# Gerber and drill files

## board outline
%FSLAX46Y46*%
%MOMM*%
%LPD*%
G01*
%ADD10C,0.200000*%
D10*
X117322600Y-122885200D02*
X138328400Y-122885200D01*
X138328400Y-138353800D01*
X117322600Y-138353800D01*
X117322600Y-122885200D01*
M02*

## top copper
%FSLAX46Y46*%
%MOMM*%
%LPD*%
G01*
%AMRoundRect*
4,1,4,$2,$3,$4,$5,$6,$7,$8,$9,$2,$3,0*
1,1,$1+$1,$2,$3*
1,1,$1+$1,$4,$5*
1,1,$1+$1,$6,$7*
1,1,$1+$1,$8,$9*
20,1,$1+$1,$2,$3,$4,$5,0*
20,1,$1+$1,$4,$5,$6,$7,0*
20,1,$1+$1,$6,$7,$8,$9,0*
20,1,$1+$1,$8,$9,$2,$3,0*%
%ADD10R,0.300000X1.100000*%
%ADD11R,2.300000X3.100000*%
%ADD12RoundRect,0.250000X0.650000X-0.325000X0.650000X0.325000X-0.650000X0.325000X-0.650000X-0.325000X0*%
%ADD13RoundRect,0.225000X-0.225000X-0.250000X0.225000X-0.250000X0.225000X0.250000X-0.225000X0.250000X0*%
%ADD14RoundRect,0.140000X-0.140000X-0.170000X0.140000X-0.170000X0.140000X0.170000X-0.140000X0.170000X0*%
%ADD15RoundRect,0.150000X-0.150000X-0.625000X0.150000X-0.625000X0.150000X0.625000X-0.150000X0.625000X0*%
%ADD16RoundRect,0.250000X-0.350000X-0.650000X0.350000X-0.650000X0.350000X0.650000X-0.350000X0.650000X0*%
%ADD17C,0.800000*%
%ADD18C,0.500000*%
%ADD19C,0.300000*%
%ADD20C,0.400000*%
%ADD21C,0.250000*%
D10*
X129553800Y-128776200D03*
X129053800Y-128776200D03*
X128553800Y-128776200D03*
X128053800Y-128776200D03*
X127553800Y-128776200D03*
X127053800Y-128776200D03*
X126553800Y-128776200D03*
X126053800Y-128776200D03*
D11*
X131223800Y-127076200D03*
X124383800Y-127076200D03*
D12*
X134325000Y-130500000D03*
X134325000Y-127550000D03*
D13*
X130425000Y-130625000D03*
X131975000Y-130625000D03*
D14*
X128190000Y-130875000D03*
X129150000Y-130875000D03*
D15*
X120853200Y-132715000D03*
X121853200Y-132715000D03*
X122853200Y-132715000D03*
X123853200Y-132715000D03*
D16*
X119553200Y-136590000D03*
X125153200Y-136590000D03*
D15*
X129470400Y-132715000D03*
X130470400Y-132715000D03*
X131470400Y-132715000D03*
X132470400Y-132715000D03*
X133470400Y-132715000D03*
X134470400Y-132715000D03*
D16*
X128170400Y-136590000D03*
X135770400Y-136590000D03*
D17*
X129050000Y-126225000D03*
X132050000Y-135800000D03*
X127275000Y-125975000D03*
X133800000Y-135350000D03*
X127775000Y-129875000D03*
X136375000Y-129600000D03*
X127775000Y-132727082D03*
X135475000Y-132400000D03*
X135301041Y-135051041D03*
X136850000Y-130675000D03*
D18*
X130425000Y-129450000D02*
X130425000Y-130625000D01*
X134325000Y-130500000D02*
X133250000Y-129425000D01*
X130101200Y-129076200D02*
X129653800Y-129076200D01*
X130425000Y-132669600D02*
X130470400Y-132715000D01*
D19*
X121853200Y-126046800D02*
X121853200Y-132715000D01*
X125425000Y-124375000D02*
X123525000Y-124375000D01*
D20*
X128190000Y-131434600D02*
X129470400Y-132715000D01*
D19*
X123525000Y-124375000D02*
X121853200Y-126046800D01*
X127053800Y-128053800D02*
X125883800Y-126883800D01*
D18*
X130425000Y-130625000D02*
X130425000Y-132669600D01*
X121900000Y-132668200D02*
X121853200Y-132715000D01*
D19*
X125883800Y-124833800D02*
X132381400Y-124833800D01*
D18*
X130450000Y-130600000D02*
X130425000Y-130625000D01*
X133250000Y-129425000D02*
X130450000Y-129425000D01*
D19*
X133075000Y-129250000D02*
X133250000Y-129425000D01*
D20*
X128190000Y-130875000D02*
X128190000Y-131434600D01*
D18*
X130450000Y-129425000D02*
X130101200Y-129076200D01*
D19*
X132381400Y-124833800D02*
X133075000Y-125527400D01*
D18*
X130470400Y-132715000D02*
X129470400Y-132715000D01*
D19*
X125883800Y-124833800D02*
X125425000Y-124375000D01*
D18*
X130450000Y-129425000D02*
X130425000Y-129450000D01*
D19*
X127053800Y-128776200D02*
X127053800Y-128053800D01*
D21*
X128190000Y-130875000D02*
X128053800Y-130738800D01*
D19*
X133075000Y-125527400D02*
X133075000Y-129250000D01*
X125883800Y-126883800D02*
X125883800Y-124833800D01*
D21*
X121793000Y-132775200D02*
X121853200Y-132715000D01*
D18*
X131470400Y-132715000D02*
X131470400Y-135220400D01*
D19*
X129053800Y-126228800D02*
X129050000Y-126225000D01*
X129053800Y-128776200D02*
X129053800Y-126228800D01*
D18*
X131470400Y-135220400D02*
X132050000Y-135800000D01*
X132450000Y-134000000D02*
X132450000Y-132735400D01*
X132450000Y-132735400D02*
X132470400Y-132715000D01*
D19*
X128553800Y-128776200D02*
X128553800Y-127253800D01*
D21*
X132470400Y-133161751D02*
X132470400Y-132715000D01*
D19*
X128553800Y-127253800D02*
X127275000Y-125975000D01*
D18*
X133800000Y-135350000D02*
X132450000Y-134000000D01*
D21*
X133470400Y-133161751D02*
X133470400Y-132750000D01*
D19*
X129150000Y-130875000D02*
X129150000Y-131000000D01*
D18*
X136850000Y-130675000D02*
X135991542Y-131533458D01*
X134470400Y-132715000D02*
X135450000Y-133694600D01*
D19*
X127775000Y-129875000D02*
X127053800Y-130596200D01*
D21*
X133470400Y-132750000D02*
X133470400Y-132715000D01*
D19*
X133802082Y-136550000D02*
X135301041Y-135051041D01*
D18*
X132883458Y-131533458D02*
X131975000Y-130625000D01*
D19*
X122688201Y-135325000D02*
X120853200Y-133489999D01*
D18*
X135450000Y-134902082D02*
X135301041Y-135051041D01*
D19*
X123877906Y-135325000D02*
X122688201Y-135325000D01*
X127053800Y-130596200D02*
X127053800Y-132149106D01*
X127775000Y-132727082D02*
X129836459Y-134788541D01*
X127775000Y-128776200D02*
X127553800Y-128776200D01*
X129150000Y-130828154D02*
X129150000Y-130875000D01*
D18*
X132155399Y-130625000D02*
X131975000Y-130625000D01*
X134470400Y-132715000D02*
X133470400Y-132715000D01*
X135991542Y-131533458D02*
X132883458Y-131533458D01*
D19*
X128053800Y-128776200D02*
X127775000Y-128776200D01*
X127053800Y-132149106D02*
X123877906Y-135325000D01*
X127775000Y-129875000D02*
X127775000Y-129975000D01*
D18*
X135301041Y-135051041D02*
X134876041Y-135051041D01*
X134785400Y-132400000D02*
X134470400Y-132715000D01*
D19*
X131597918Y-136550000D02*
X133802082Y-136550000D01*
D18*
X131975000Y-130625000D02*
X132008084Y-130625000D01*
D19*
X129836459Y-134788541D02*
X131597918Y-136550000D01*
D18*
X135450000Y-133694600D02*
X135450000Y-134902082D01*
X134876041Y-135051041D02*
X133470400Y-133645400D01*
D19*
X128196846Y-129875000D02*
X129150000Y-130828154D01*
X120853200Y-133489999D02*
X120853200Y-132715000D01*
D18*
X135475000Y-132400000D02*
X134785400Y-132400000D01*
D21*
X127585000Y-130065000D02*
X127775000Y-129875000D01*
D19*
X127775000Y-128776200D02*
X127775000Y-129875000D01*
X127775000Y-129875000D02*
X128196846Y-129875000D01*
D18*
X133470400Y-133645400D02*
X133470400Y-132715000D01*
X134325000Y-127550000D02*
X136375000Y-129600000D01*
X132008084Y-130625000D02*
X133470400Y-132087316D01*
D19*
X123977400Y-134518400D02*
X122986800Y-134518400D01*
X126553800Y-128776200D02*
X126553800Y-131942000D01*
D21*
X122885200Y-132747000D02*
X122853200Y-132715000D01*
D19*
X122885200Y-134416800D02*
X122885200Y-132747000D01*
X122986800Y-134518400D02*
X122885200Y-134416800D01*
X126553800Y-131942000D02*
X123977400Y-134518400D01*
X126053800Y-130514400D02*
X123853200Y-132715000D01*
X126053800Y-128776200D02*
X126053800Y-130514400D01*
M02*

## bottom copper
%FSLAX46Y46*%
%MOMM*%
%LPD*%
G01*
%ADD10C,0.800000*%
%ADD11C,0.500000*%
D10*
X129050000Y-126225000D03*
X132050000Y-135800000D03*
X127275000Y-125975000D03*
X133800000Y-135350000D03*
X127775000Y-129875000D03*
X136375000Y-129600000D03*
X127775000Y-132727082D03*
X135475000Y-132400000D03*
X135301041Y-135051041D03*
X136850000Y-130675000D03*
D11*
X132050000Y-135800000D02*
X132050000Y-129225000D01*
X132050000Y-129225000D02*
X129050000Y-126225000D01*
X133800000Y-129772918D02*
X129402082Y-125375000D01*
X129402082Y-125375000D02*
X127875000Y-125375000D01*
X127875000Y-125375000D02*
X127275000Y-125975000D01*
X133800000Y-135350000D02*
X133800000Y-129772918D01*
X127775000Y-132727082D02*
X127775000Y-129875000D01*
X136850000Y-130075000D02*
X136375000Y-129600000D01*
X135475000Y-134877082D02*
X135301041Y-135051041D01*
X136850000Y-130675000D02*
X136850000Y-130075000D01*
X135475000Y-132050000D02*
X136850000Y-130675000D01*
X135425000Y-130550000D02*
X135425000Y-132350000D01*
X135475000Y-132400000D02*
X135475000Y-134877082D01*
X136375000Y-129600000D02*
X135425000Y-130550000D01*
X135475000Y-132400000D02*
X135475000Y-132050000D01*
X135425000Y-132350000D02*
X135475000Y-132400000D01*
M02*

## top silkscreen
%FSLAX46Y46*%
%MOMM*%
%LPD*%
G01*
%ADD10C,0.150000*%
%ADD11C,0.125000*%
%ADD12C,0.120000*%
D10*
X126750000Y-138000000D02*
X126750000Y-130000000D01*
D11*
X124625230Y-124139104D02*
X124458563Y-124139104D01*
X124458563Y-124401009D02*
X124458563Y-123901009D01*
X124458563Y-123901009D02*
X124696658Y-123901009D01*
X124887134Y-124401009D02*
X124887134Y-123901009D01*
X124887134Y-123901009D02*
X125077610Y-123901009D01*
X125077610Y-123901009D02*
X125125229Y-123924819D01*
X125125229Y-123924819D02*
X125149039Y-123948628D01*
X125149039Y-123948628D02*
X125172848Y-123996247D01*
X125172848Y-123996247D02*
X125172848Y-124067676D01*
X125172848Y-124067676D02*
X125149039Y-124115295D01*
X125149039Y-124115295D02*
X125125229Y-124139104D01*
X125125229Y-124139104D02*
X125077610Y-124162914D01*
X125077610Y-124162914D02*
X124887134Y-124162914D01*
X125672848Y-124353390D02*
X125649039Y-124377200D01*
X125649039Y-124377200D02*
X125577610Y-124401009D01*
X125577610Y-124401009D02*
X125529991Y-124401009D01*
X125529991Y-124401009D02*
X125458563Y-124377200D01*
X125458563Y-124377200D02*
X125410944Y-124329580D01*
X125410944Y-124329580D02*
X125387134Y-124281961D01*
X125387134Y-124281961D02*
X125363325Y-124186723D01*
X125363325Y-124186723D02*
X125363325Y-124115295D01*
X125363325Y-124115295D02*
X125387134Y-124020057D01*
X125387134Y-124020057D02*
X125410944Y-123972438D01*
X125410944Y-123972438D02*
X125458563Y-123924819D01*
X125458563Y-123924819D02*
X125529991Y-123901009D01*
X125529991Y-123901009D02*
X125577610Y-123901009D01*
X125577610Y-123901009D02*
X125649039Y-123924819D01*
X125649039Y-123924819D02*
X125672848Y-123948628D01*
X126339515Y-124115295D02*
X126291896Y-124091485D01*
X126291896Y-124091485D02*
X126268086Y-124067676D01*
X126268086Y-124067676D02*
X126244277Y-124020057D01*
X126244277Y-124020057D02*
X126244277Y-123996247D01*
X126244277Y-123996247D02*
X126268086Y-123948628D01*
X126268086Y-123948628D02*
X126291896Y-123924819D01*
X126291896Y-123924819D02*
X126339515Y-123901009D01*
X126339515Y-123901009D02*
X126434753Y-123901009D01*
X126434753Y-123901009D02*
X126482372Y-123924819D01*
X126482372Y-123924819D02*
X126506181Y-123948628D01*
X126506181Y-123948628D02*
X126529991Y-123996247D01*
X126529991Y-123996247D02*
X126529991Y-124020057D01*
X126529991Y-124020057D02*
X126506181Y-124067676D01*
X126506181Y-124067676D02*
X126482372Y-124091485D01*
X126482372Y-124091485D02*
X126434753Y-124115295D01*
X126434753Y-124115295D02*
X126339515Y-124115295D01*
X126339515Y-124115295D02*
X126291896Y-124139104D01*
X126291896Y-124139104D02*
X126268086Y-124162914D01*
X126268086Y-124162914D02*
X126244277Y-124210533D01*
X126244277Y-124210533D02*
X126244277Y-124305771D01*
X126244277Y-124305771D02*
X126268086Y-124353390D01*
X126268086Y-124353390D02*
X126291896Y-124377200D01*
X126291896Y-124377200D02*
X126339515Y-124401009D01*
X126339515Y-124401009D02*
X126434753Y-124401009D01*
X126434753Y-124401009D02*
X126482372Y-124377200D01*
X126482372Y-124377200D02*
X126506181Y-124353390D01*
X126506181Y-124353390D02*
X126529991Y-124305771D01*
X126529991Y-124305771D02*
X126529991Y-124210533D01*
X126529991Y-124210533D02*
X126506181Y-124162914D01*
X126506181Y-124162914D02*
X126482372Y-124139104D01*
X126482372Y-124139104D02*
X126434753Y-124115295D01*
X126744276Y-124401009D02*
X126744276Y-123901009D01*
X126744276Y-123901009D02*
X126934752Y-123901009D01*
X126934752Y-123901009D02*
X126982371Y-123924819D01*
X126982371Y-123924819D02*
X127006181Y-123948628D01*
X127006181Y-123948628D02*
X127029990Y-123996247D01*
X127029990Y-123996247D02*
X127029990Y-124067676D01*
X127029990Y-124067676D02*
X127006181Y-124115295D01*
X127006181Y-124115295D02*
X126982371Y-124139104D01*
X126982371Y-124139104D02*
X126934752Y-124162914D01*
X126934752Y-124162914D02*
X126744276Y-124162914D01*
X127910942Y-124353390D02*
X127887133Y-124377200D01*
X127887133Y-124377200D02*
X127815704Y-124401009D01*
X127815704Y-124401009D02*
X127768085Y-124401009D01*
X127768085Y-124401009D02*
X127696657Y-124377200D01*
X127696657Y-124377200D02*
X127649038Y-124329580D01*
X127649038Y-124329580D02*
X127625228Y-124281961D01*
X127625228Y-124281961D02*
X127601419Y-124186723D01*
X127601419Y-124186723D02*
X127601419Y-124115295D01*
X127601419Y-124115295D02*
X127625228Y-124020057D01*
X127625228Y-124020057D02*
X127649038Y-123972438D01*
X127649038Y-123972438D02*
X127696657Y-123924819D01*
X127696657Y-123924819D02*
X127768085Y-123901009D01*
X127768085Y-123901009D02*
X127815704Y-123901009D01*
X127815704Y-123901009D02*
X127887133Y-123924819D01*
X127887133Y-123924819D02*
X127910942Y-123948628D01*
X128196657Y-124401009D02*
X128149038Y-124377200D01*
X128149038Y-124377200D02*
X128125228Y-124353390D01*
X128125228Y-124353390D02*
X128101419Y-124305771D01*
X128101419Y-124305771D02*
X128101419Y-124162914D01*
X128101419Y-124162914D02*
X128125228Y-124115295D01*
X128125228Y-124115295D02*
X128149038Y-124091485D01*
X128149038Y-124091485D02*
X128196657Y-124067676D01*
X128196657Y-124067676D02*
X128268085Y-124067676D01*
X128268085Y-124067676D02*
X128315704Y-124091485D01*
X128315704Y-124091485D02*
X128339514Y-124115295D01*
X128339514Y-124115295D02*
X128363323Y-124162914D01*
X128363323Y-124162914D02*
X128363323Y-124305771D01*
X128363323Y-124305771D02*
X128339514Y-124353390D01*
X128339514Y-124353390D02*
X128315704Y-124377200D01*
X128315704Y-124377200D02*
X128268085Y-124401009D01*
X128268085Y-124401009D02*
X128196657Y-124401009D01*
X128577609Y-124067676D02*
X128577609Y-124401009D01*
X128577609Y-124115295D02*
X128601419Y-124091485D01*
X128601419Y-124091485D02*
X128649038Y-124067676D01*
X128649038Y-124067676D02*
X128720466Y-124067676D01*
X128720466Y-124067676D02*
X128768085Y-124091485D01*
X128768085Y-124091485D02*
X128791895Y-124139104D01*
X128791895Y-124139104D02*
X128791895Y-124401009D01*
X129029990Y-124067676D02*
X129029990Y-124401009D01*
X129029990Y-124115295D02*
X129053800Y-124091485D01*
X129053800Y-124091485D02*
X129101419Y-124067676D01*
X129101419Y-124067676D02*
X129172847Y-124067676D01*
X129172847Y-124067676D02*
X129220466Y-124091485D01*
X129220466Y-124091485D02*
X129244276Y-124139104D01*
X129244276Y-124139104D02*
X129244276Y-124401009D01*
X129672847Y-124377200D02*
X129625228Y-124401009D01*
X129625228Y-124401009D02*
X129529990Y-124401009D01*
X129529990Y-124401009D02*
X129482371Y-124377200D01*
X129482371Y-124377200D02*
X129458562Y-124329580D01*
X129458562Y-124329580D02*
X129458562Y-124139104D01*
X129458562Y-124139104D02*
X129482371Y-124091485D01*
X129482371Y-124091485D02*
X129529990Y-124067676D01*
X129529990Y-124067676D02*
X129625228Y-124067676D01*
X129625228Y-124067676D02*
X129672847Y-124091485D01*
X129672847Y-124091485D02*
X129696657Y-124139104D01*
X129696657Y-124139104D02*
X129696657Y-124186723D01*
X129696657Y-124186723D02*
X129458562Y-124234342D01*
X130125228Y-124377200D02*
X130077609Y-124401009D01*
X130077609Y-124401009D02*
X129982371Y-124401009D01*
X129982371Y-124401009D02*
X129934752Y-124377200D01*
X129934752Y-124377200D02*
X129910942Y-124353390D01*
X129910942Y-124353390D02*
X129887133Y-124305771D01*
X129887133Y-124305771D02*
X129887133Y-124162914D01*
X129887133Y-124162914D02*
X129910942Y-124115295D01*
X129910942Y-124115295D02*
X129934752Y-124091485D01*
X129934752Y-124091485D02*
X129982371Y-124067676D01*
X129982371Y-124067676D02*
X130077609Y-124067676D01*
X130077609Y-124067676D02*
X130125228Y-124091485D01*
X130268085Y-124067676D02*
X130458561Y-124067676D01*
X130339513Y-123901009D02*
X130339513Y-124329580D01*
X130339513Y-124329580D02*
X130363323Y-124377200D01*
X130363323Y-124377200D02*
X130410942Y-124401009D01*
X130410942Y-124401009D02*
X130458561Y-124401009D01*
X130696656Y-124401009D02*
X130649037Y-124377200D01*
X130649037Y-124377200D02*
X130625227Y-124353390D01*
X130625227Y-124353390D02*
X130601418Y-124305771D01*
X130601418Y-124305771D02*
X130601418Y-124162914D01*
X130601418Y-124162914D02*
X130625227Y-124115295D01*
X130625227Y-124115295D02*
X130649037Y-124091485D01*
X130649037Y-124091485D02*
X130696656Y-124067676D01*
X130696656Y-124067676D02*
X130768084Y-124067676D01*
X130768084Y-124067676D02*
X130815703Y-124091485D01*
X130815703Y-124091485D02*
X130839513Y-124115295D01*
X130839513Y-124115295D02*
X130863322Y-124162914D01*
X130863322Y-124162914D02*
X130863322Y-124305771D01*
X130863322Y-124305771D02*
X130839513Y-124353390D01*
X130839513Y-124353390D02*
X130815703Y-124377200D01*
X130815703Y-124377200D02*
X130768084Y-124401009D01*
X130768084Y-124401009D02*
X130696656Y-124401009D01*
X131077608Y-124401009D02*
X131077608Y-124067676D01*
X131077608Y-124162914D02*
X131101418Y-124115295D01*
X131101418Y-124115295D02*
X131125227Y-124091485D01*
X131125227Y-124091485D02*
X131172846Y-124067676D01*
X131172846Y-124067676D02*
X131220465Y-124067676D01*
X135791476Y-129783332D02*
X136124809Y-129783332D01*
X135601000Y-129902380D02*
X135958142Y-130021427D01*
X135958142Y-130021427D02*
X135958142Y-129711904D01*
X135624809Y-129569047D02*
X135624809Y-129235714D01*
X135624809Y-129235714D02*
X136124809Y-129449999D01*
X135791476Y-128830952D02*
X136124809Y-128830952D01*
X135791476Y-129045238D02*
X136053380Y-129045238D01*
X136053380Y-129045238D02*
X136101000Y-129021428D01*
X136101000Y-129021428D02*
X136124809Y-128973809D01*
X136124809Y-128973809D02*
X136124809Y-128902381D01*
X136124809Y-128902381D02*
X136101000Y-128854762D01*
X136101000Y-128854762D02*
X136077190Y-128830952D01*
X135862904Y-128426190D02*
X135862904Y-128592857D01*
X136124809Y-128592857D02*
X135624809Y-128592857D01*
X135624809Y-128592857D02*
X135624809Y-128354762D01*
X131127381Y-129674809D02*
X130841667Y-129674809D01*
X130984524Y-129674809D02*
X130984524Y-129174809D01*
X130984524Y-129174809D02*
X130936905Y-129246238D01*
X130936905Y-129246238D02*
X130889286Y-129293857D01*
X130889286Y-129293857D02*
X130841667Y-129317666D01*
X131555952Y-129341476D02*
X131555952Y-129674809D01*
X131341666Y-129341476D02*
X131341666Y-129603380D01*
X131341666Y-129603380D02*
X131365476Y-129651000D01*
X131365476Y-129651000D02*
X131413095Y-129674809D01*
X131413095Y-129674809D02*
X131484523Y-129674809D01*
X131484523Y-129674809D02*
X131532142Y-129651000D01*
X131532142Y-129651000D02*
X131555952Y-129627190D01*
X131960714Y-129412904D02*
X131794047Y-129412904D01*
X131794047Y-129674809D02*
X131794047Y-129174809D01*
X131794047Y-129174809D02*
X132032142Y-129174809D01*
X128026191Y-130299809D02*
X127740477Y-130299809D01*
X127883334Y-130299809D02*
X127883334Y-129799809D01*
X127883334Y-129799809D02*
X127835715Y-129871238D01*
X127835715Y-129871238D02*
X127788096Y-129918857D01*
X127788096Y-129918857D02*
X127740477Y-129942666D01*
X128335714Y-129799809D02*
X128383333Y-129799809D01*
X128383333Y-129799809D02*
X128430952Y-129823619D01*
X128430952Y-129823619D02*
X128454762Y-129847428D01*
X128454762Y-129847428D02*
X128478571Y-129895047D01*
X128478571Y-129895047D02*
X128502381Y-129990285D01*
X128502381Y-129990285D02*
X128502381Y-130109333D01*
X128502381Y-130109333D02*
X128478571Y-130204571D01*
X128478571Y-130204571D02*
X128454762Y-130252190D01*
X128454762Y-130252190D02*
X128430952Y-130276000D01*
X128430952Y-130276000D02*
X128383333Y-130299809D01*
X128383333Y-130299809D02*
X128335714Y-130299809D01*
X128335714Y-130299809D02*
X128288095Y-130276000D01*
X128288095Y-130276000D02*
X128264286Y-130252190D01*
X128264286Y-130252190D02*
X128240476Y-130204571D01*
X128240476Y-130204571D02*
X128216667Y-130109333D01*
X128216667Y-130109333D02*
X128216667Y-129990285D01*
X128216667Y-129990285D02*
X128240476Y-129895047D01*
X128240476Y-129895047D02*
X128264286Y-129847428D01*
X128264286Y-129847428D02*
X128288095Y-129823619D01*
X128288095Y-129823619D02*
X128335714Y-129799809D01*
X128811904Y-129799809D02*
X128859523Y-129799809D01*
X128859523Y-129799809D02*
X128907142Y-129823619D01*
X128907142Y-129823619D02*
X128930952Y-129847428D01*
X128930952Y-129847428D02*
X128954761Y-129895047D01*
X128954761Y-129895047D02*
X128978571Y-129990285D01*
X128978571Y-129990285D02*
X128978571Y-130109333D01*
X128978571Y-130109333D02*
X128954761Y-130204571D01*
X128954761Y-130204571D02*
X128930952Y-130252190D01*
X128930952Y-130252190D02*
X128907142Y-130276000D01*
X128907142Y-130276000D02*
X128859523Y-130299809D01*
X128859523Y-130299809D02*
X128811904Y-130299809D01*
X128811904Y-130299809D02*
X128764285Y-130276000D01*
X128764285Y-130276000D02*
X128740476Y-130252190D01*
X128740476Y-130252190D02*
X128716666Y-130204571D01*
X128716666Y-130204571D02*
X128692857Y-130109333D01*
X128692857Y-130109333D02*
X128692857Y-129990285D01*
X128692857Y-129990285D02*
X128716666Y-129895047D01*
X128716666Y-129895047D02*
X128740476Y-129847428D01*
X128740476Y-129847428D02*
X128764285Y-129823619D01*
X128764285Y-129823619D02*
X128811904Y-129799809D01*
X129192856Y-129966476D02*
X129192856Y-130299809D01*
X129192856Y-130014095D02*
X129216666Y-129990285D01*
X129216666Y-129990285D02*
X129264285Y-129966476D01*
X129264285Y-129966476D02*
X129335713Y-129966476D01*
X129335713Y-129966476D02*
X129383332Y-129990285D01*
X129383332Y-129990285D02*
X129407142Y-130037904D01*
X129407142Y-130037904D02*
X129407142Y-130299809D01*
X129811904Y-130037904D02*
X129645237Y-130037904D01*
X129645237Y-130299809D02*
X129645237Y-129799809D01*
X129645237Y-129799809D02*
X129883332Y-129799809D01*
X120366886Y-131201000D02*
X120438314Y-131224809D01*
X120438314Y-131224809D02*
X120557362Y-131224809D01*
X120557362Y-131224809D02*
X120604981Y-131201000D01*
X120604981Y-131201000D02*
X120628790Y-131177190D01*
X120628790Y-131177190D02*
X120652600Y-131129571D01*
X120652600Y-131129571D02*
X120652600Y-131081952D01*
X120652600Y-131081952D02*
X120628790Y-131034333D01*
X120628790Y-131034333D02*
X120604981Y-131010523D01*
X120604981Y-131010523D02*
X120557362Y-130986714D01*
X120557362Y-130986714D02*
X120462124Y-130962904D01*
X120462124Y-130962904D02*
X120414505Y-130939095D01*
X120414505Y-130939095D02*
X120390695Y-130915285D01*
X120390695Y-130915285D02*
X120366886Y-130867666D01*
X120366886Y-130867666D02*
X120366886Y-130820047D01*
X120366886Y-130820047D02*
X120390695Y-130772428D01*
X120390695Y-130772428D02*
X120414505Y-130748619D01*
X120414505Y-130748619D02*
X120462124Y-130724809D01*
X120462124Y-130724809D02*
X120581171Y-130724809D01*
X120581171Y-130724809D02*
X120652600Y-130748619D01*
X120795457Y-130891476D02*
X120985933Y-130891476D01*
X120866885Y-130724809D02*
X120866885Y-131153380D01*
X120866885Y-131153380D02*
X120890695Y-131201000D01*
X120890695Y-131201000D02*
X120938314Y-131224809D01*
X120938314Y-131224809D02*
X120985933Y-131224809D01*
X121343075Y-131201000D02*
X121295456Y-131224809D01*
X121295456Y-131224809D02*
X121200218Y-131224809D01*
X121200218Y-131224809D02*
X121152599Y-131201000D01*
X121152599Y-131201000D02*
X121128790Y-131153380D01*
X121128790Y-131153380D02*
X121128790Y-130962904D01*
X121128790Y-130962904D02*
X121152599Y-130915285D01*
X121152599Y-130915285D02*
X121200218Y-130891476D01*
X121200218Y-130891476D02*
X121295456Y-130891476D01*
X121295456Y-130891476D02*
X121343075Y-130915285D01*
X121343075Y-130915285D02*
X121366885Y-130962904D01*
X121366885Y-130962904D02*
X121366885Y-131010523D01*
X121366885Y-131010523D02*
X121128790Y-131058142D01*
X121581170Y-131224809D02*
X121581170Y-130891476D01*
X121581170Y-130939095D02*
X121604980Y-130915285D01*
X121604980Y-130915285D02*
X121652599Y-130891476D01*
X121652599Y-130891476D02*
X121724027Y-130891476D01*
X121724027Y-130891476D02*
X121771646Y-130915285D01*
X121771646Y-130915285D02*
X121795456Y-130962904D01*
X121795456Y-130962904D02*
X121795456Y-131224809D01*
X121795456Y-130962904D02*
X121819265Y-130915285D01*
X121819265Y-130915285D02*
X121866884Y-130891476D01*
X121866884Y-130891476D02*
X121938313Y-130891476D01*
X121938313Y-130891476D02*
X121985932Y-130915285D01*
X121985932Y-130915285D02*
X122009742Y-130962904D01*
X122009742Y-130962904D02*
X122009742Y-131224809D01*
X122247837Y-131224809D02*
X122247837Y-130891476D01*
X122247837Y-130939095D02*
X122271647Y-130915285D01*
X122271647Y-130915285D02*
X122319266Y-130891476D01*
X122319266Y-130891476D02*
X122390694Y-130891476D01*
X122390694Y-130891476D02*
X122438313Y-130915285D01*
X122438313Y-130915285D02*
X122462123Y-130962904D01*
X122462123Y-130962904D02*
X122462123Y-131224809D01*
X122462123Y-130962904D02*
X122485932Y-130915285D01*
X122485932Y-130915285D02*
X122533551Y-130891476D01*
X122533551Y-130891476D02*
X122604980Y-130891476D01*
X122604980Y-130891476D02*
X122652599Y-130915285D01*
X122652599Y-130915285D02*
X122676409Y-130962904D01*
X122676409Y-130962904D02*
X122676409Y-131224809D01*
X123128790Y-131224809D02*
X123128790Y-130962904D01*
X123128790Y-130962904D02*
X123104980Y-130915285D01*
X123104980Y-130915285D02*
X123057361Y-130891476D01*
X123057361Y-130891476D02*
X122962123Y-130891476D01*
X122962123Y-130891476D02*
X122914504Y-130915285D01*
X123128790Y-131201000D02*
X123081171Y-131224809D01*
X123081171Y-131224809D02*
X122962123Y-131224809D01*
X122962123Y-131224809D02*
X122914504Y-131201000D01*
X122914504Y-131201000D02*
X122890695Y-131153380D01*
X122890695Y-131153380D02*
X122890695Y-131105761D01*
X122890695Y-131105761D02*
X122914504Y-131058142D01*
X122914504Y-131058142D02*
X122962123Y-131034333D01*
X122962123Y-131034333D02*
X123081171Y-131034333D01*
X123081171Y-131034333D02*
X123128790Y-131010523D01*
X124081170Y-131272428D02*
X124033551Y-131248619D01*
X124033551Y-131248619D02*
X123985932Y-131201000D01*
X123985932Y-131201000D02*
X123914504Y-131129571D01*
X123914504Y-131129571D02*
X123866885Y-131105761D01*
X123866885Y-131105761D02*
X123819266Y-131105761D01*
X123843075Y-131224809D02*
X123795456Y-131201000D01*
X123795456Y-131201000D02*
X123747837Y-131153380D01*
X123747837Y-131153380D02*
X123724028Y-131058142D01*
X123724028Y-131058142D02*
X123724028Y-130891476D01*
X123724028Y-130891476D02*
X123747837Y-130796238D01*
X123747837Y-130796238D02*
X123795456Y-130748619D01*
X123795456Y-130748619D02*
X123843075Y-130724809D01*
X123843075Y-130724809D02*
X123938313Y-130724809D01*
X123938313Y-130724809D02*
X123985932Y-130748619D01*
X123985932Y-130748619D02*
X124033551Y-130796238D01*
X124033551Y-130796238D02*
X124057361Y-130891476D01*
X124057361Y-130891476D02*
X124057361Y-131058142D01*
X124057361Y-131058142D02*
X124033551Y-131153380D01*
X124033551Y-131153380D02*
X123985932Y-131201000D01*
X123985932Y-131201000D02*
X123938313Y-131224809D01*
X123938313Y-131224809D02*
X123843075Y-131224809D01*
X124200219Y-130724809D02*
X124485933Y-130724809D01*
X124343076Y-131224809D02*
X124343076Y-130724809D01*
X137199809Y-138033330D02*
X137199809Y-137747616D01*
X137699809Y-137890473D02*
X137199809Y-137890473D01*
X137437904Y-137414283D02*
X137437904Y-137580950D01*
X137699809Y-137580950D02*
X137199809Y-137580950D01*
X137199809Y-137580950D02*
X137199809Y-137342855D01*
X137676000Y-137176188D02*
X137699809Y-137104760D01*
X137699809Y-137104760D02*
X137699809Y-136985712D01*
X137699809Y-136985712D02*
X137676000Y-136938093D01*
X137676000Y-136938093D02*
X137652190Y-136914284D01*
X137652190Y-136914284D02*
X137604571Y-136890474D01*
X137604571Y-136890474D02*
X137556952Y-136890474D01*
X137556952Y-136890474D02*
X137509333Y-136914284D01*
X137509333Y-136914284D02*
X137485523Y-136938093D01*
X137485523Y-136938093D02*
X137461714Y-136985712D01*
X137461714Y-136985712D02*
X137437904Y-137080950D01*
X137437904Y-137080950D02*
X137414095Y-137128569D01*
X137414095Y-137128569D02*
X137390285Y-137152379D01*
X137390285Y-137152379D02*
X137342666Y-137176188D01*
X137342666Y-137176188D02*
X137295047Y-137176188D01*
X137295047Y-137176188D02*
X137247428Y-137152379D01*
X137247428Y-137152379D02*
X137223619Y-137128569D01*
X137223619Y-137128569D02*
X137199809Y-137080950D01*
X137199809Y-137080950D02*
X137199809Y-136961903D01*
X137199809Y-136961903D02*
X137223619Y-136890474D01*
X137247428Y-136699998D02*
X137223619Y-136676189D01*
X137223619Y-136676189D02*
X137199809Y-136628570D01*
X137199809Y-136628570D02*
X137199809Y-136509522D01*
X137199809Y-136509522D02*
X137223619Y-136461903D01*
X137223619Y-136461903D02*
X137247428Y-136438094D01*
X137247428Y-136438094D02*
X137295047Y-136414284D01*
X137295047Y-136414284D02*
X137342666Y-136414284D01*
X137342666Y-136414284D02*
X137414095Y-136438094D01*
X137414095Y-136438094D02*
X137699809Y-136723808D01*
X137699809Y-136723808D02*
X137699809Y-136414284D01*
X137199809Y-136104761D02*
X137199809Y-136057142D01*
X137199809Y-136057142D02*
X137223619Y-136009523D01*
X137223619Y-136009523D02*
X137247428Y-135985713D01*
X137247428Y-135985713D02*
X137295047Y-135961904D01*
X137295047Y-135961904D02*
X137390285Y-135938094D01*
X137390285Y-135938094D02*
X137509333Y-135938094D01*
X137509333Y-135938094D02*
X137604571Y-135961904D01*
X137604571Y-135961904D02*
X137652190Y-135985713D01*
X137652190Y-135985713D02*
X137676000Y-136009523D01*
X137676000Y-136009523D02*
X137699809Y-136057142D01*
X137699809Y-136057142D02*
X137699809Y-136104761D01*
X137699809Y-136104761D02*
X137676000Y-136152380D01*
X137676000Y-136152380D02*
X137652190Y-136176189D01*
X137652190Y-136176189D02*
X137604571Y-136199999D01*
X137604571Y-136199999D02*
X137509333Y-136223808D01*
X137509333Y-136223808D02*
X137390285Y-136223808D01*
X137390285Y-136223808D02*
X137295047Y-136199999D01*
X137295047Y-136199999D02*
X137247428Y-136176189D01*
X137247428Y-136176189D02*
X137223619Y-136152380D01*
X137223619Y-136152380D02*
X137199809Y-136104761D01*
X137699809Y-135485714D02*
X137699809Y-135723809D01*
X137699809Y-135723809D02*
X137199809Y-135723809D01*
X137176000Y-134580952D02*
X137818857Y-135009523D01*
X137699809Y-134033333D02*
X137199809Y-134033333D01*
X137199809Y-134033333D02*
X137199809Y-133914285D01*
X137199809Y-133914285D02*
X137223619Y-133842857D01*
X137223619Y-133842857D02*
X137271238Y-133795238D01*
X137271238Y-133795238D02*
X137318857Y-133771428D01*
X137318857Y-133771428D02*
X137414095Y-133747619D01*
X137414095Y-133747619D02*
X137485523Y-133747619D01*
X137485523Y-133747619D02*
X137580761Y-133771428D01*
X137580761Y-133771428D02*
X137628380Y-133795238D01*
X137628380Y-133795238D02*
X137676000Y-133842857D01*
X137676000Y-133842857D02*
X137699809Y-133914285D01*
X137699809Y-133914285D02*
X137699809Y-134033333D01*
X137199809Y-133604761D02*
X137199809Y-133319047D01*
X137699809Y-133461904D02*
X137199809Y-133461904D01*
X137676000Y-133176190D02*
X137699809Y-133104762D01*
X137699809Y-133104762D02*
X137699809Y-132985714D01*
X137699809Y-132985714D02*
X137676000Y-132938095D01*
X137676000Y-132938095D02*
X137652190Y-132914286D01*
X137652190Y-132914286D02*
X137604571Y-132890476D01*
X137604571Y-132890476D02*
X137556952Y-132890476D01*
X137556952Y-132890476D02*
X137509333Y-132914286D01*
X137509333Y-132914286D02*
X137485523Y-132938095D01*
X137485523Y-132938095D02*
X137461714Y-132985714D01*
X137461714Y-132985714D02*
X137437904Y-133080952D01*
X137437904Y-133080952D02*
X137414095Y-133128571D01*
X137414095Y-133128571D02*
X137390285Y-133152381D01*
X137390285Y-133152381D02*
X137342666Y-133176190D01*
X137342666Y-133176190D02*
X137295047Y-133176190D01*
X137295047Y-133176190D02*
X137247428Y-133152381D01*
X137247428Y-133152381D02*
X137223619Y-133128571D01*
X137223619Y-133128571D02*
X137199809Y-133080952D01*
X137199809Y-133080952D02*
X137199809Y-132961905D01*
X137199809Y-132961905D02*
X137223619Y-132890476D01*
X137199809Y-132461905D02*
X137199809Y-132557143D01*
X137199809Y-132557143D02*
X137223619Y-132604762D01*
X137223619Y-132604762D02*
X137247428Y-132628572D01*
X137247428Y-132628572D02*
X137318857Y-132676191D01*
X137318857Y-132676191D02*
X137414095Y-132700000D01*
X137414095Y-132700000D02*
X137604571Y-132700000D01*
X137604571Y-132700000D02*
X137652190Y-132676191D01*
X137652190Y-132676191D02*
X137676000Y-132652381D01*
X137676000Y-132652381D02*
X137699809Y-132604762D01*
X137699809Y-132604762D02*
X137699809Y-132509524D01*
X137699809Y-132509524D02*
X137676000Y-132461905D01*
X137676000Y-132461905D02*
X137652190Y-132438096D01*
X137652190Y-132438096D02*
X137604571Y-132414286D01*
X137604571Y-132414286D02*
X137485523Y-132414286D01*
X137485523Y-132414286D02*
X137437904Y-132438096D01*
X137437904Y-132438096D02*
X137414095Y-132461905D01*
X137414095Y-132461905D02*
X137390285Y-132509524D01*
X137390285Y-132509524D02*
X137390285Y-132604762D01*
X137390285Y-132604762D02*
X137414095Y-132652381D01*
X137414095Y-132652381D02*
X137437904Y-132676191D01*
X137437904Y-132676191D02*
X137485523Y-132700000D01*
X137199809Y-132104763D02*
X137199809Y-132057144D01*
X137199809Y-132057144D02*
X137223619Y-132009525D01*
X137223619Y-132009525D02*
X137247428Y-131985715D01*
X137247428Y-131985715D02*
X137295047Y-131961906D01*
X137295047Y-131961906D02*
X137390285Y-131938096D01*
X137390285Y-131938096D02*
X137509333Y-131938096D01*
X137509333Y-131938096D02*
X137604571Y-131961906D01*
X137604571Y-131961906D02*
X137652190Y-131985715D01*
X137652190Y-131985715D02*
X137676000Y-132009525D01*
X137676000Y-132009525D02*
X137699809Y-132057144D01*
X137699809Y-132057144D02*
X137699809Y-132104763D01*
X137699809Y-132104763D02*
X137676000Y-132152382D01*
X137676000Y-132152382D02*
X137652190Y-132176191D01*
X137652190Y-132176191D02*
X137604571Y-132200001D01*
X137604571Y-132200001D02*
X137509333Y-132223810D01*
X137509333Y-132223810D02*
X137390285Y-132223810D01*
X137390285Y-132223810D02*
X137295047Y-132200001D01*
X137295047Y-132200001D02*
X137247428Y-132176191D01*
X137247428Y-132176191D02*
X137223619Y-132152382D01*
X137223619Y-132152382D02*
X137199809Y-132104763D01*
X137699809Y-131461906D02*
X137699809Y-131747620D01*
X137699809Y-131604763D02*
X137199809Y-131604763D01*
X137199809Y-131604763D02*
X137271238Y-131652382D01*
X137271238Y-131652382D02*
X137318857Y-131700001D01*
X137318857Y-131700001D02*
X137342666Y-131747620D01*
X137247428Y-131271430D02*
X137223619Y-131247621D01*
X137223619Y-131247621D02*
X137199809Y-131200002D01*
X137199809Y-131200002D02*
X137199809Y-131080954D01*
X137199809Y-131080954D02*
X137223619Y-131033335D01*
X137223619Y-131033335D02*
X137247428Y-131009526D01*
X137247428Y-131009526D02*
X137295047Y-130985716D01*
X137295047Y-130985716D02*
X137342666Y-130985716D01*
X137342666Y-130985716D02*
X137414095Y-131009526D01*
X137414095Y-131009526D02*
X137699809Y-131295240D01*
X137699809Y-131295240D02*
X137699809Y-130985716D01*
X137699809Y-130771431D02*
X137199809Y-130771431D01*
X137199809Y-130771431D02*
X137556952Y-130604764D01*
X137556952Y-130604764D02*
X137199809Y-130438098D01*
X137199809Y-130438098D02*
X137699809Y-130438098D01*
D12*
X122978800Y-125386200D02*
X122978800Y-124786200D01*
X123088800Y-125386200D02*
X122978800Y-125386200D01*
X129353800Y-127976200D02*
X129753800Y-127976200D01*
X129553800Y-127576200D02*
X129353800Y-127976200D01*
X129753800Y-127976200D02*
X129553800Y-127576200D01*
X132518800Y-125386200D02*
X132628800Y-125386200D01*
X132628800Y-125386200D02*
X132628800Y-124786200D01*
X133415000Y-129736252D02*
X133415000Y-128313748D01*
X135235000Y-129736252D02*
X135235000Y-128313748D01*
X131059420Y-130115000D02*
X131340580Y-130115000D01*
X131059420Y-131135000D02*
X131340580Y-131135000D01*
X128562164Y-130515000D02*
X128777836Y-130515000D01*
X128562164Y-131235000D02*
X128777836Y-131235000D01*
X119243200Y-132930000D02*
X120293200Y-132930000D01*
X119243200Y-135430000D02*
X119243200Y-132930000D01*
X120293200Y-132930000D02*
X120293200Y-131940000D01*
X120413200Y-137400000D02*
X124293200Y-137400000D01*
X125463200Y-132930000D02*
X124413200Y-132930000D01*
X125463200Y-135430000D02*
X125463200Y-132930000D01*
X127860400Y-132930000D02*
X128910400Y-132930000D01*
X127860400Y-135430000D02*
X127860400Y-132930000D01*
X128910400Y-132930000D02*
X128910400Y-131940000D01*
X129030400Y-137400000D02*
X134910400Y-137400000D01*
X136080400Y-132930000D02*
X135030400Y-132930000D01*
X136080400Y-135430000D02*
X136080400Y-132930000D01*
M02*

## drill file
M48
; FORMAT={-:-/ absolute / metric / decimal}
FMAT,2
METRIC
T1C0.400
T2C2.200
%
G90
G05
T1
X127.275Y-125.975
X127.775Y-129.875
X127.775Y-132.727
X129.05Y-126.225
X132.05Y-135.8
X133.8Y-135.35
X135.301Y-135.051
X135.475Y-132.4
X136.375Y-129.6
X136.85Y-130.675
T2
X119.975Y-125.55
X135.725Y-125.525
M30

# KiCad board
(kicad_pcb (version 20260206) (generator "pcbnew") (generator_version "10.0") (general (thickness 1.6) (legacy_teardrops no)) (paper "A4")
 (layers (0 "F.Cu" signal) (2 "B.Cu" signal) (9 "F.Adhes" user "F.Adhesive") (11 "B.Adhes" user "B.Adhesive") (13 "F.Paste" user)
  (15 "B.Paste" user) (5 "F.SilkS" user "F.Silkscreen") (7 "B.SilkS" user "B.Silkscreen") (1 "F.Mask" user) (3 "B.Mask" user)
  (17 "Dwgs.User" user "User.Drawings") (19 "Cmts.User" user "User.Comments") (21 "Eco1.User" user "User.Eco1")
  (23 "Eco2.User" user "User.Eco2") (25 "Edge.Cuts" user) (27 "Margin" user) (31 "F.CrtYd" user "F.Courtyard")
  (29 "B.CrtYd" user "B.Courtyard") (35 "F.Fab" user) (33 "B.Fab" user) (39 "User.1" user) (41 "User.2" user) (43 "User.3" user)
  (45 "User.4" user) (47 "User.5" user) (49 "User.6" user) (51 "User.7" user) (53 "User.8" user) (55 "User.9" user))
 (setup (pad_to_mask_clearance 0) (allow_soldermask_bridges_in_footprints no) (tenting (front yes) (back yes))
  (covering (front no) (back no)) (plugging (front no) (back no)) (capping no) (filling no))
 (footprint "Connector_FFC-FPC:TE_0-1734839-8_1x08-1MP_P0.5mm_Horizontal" (layer "F.Cu") (at 127.8038 127.4262 180)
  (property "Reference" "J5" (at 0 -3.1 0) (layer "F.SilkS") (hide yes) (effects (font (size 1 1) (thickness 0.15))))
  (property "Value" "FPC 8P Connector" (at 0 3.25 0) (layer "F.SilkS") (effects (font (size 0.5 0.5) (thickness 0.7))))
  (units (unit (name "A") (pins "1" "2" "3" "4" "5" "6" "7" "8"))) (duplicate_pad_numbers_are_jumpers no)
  (fp_line (start 4.825 2.04) (end 4.825 2.64) (stroke (width 0.12) (type solid)) (layer "F.SilkS"))
  (fp_line (start 4.715 2.04) (end 4.825 2.04) (stroke (width 0.12) (type solid)) (layer "F.SilkS"))
  (fp_line (start -1.55 -0.55) (end -1.95 -0.55) (stroke (width 0.12) (type solid)) (layer "F.SilkS"))
  (fp_line (start -1.75 -0.15) (end -1.55 -0.55) (stroke (width 0.12) (type solid)) (layer "F.SilkS"))
  (fp_line (start -1.95 -0.55) (end -1.75 -0.15) (stroke (width 0.12) (type solid)) (layer "F.SilkS"))
  (fp_line (start -4.715 2.04) (end -4.825 2.04) (stroke (width 0.12) (type solid)) (layer "F.SilkS"))
  (fp_line (start -4.825 2.04) (end -4.825 2.64) (stroke (width 0.12) (type solid)) (layer "F.SilkS"))
  (pad "1" smd rect (at -1.75 -1.35 180) (size 0.3 1.1) (layers "F.Cu" "F.Mask" "F.Paste") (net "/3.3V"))
  (pad "2" smd rect (at -1.25 -1.35 180) (size 0.3 1.1) (layers "F.Cu" "F.Mask" "F.Paste") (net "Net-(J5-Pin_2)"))
  (pad "3" smd rect (at -0.75 -1.35 180) (size 0.3 1.1) (layers "F.Cu" "F.Mask" "F.Paste") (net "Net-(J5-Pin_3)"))
  (pad "4" smd rect (at -0.25 -1.35 180) (size 0.3 1.1) (layers "F.Cu" "F.Mask" "F.Paste") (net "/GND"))
  (pad "5" smd rect (at 0.25 -1.35 180) (size 0.3 1.1) (layers "F.Cu" "F.Mask" "F.Paste") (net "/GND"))
  (pad "6" smd rect (at 0.75 -1.35 180) (size 0.3 1.1) (layers "F.Cu" "F.Mask" "F.Paste") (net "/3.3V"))
  (pad "7" smd rect (at 1.25 -1.35 180) (size 0.3 1.1) (layers "F.Cu" "F.Mask" "F.Paste") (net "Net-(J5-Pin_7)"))
  (pad "8" smd rect (at 1.75 -1.35 180) (size 0.3 1.1) (layers "F.Cu" "F.Mask" "F.Paste") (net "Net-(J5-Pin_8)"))
  (pad "MP" smd rect (at -3.42 0.35 180) (size 2.3 3.1) (layers "F.Cu" "F.Mask" "F.Paste"))
  (pad "MP" smd rect (at 3.42 0.35 180) (size 2.3 3.1) (layers "F.Cu" "F.Mask" "F.Paste")))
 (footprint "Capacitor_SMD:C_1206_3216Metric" (layer "F.Cu") (at 134.325 129.025 90)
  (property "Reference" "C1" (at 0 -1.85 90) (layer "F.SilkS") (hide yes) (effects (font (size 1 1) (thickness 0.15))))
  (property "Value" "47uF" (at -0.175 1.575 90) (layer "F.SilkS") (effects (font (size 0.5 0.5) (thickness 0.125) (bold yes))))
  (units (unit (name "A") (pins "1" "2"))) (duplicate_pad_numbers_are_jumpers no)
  (fp_line (start -0.711252 -0.91) (end 0.711252 -0.91) (stroke (width 0.12) (type solid)) (layer "F.SilkS"))
  (fp_line (start -0.711252 0.91) (end 0.711252 0.91) (stroke (width 0.12) (type solid)) (layer "F.SilkS"))
  (pad "1" smd roundrect (at -1.475 0 90) (size 1.15 1.8) (layers "F.Cu" "F.Mask" "F.Paste") (roundrect_rratio 0.217391) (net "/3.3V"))
  (pad "2" smd roundrect (at 1.475 0 90) (size 1.15 1.8) (layers "F.Cu" "F.Mask" "F.Paste") (roundrect_rratio 0.217391) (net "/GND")))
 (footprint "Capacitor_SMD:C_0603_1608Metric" (layer "F.Cu") (at 131.2 130.625)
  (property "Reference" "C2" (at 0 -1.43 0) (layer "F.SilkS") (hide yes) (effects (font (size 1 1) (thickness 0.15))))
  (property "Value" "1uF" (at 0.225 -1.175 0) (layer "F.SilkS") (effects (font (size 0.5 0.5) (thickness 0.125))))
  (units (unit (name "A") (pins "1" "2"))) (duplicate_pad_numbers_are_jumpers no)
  (fp_line (start -0.14058 -0.51) (end 0.14058 -0.51) (stroke (width 0.12) (type solid)) (layer "F.SilkS"))
  (fp_line (start -0.14058 0.51) (end 0.14058 0.51) (stroke (width 0.12) (type solid)) (layer "F.SilkS"))
  (pad "1" smd roundrect (at -0.775 0) (size 0.9 0.95) (layers "F.Cu" "F.Mask" "F.Paste") (roundrect_rratio 0.25) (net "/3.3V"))
  (pad "2" smd roundrect (at 0.775 0) (size 0.9 0.95) (layers "F.Cu" "F.Mask" "F.Paste") (roundrect_rratio 0.25) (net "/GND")))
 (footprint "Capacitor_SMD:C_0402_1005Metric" (layer "F.Cu") (at 128.67 130.875)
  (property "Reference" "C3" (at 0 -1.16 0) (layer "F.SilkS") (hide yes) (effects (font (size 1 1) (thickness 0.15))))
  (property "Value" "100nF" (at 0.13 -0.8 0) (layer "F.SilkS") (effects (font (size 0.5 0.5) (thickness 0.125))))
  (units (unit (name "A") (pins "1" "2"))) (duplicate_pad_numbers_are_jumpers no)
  (fp_line (start -0.107836 -0.36) (end 0.107836 -0.36) (stroke (width 0.12) (type solid)) (layer "F.SilkS"))
  (fp_line (start -0.107836 0.36) (end 0.107836 0.36) (stroke (width 0.12) (type solid)) (layer "F.SilkS"))
  (pad "1" smd roundrect (at -0.48 0) (size 0.56 0.62) (layers "F.Cu" "F.Mask" "F.Paste") (roundrect_rratio 0.25) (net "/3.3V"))
  (pad "2" smd roundrect (at 0.48 0) (size 0.56 0.62) (layers "F.Cu" "F.Mask" "F.Paste") (roundrect_rratio 0.25) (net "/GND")))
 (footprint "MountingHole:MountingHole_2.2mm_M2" (layer "F.Cu") (at 119.975 125.55)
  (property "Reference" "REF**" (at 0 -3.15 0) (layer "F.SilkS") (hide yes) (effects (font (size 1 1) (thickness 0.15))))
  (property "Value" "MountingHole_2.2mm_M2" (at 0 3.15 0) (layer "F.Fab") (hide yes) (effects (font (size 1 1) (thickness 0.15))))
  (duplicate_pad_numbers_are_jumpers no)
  (pad "" np_thru_hole circle (at 0 0) (size 2.2 2.2) (drill 2.2) (layers "*.Cu" "*.Mask")))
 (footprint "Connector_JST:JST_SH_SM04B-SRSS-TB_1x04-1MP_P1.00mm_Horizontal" (layer "F.Cu") (at 122.3532 134.715)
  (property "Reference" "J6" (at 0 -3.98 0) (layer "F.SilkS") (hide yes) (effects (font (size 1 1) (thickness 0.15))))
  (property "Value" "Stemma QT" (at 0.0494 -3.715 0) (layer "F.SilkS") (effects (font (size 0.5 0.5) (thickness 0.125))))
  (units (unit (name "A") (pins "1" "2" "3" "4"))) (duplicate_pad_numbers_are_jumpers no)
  (fp_line (start -3.11 -1.785) (end -2.06 -1.785) (stroke (width 0.12) (type solid)) (layer "F.SilkS"))
  (fp_line (start -3.11 0.715) (end -3.11 -1.785) (stroke (width 0.12) (type solid)) (layer "F.SilkS"))
  (fp_line (start -2.06 -1.785) (end -2.06 -2.775) (stroke (width 0.12) (type solid)) (layer "F.SilkS"))
  (fp_line (start -1.94 2.685) (end 1.94 2.685) (stroke (width 0.12) (type solid)) (layer "F.SilkS"))
  (fp_line (start 3.11 -1.785) (end 2.06 -1.785) (stroke (width 0.12) (type solid)) (layer "F.SilkS"))
  (fp_line (start 3.11 0.715) (end 3.11 -1.785) (stroke (width 0.12) (type solid)) (layer "F.SilkS"))
  (pad "1" smd roundrect (at -1.5 -2) (size 0.6 1.55) (layers "F.Cu" "F.Mask" "F.Paste") (roundrect_rratio 0.25) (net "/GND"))
  (pad "2" smd roundrect (at -0.5 -2) (size 0.6 1.55) (layers "F.Cu" "F.Mask" "F.Paste") (roundrect_rratio 0.25) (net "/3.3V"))
  (pad "3" smd roundrect (at 0.5 -2) (size 0.6 1.55) (layers "F.Cu" "F.Mask" "F.Paste") (roundrect_rratio 0.25) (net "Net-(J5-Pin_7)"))
  (pad "4" smd roundrect (at 1.5 -2) (size 0.6 1.55) (layers "F.Cu" "F.Mask" "F.Paste") (roundrect_rratio 0.25) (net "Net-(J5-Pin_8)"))
  (pad "MP" smd roundrect (at -2.8 1.875) (size 1.2 1.8) (layers "F.Cu" "F.Mask" "F.Paste") (roundrect_rratio 0.2083333333))
  (pad "MP" smd roundrect (at 2.8 1.875) (size 1.2 1.8) (layers "F.Cu" "F.Mask" "F.Paste") (roundrect_rratio 0.2083333333)))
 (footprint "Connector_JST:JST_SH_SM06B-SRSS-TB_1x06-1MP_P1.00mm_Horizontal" (layer "F.Cu") (at 131.9704 134.715)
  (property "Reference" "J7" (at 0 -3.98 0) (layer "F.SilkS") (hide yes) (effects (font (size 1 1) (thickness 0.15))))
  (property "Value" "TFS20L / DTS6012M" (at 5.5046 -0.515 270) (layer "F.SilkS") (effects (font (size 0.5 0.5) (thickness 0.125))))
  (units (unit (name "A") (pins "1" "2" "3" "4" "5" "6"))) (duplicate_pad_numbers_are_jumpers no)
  (fp_line (start -4.11 -1.785) (end -3.06 -1.785) (stroke (width 0.12) (type solid)) (layer "F.SilkS"))
  (fp_line (start -4.11 0.715) (end -4.11 -1.785) (stroke (width 0.12) (type solid)) (layer "F.SilkS"))
  (fp_line (start -3.06 -1.785) (end -3.06 -2.775) (stroke (width 0.12) (type solid)) (layer "F.SilkS"))
  (fp_line (start -2.94 2.685) (end 2.94 2.685) (stroke (width 0.12) (type solid)) (layer "F.SilkS"))
  (fp_line (start 4.11 -1.785) (end 3.06 -1.785) (stroke (width 0.12) (type solid)) (layer "F.SilkS"))
  (fp_line (start 4.11 0.715) (end 4.11 -1.785) (stroke (width 0.12) (type solid)) (layer "F.SilkS"))
  (pad "1" smd roundrect (at -2.5 -2) (size 0.6 1.55) (layers "F.Cu" "F.Mask" "F.Paste") (roundrect_rratio 0.25) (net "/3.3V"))
  (pad "2" smd roundrect (at -1.5 -2) (size 0.6 1.55) (layers "F.Cu" "F.Mask" "F.Paste") (roundrect_rratio 0.25) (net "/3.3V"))
  (pad "3" smd roundrect (at -0.5 -2) (size 0.6 1.55) (layers "F.Cu" "F.Mask" "F.Paste") (roundrect_rratio 0.25) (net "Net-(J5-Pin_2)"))
  (pad "4" smd roundrect (at 0.5 -2) (size 0.6 1.55) (layers "F.Cu" "F.Mask" "F.Paste") (roundrect_rratio 0.25) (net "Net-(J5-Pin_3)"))
  (pad "5" smd roundrect (at 1.5 -2) (size 0.6 1.55) (layers "F.Cu" "F.Mask" "F.Paste") (roundrect_rratio 0.25) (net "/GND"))
  (pad "6" smd roundrect (at 2.5 -2) (size 0.6 1.55) (layers "F.Cu" "F.Mask" "F.Paste") (roundrect_rratio 0.25) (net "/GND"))
  (pad "MP" smd roundrect (at -3.8 1.875) (size 1.2 1.8) (layers "F.Cu" "F.Mask" "F.Paste") (roundrect_rratio 0.2083333333))
  (pad "MP" smd roundrect (at 3.8 1.875) (size 1.2 1.8) (layers "F.Cu" "F.Mask" "F.Paste") (roundrect_rratio 0.2083333333)))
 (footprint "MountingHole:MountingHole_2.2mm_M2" (layer "F.Cu") (at 135.725 125.525)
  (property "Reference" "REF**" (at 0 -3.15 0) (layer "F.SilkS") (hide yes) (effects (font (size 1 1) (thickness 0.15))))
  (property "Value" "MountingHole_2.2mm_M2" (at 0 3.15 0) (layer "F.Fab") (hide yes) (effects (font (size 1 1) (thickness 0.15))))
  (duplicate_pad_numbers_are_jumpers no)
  (pad "" np_thru_hole circle (at 0 0) (size 2.2 2.2) (drill 2.2) (layers "*.Cu" "*.Mask")))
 (gr_line (start 126.75 138) (end 126.75 130) (stroke (width 0.15) (type default)) (layer "F.SilkS"))
 (gr_rect (start 117.3226 122.8852) (end 138.3284 138.3538) (stroke (width 0.2) (type default)) (fill no) (layer "Edge.Cuts"))
 (segment (start 130.425 129.45) (end 130.425 130.625) (width 0.5) (layer "F.Cu") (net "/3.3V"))
 (segment (start 134.325 130.5) (end 133.25 129.425) (width 0.5) (layer "F.Cu") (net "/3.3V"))
 (segment (start 130.1012 129.0762) (end 129.6538 129.0762) (width 0.5) (layer "F.Cu") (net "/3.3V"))
 (segment (start 130.425 132.6696) (end 130.4704 132.715) (width 0.5) (layer "F.Cu") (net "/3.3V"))
 (segment (start 121.8532 126.0468) (end 121.8532 132.715) (width 0.3) (layer "F.Cu") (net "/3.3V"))
 (segment (start 125.425 124.375) (end 123.525 124.375) (width 0.3) (layer "F.Cu") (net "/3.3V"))
 (segment (start 128.19 131.4346) (end 129.4704 132.715) (width 0.4) (layer "F.Cu") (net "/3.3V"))
 (segment (start 123.525 124.375) (end 121.8532 126.0468) (width 0.3) (layer "F.Cu") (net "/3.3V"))
 (segment (start 127.0538 128.0538) (end 125.8838 126.8838) (width 0.3) (layer "F.Cu") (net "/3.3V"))
 (segment (start 130.425 130.625) (end 130.425 132.6696) (width 0.5) (layer "F.Cu") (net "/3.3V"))
 (segment (start 121.9 132.6682) (end 121.8532 132.715) (width 0.5) (layer "F.Cu") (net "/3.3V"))
 (segment (start 125.8838 124.8338) (end 132.3814 124.8338) (width 0.3) (layer "F.Cu") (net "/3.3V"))
 (segment (start 130.45 130.6) (end 130.425 130.625) (width 0.5) (layer "F.Cu") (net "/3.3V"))
 (segment (start 133.25 129.425) (end 130.45 129.425) (width 0.5) (layer "F.Cu") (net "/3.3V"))
 (segment (start 133.075 129.25) (end 133.25 129.425) (width 0.3) (layer "F.Cu") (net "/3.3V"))
 (segment (start 128.19 130.875) (end 128.19 131.4346) (width 0.4) (layer "F.Cu") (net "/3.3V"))
 (segment (start 130.45 129.425) (end 130.1012 129.0762) (width 0.5) (layer "F.Cu") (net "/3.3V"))
 (segment (start 132.3814 124.8338) (end 133.075 125.5274) (width 0.3) (layer "F.Cu") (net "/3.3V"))
 (segment (start 130.4704 132.715) (end 129.4704 132.715) (width 0.5) (layer "F.Cu") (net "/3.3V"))
 (segment (start 125.8838 124.8338) (end 125.425 124.375) (width 0.3) (layer "F.Cu") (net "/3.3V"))
 (segment (start 130.45 129.425) (end 130.425 129.45) (width 0.5) (layer "F.Cu") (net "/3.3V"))
 (segment (start 127.0538 128.7762) (end 127.0538 128.0538) (width 0.3) (layer "F.Cu") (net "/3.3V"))
 (segment (start 128.19 130.875) (end 128.0538 130.7388) (width 0.25) (layer "F.Cu") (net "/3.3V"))
 (segment (start 133.075 125.5274) (end 133.075 129.25) (width 0.3) (layer "F.Cu") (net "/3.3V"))
 (segment (start 125.8838 126.8838) (end 125.8838 124.8338) (width 0.3) (layer "F.Cu") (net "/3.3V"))
 (segment (start 121.793 132.7752) (end 121.8532 132.715) (width 0.25) (layer "F.Cu") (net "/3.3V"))
 (segment (start 131.4704 132.715) (end 131.4704 135.2204) (width 0.5) (layer "F.Cu") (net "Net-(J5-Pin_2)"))
 (segment (start 129.0538 126.2288) (end 129.05 126.225) (width 0.3) (layer "F.Cu") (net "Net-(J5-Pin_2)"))
 (segment (start 129.0538 128.7762) (end 129.0538 126.2288) (width 0.3) (layer "F.Cu") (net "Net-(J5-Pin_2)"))
 (segment (start 131.4704 135.2204) (end 132.05 135.8) (width 0.5) (layer "F.Cu") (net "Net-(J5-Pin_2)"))
 (via (at 129.05 126.225) (size 0.8) (drill 0.4) (layers "F.Cu" "B.Cu") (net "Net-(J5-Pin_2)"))
 (via (at 132.05 135.8) (size 0.8) (drill 0.4) (layers "F.Cu" "B.Cu") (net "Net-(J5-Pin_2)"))
 (segment (start 132.05 135.8) (end 132.05 129.225) (width 0.5) (layer "B.Cu") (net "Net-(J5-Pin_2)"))
 (segment (start 132.05 129.225) (end 129.05 126.225) (width 0.5) (layer "B.Cu") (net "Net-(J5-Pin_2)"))
 (segment (start 132.45 134) (end 132.45 132.7354) (width 0.5) (layer "F.Cu") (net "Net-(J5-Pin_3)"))
 (segment (start 132.45 132.7354) (end 132.4704 132.715) (width 0.5) (layer "F.Cu") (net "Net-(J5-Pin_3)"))
 (segment (start 128.5538 128.7762) (end 128.5538 127.2538) (width 0.3) (layer "F.Cu") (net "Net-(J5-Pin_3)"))
 (segment (start 132.4704 133.161751) (end 132.4704 132.715) (width 0.25) (layer "F.Cu") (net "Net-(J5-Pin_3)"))
 (segment (start 128.5538 127.2538) (end 127.275 125.975) (width 0.3) (layer "F.Cu") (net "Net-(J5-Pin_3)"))
 (segment (start 133.8 135.35) (end 132.45 134) (width 0.5) (layer "F.Cu") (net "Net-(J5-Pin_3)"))
 (via (at 127.275 125.975) (size 0.8) (drill 0.4) (layers "F.Cu" "B.Cu") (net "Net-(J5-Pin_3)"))
 (via (at 133.8 135.35) (size 0.8) (drill 0.4) (layers "F.Cu" "B.Cu") (capping no) (covering (front no) (back no))
  (plugging (front no) (back no)) (filling no) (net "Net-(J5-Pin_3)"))
 (segment (start 133.8 129.772918) (end 129.402082 125.375) (width 0.5) (layer "B.Cu") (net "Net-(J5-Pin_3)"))
 (segment (start 129.402082 125.375) (end 127.875 125.375) (width 0.5) (layer "B.Cu") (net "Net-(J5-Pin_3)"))
 (segment (start 127.875 125.375) (end 127.275 125.975) (width 0.5) (layer "B.Cu") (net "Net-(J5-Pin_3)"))
 (segment (start 133.8 135.35) (end 133.8 129.772918) (width 0.5) (layer "B.Cu") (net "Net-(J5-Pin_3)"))
 (segment (start 133.4704 133.161751) (end 133.4704 132.75) (width 0.25) (layer "F.Cu") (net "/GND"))
 (segment (start 129.15 130.875) (end 129.15 131) (width 0.3) (layer "F.Cu") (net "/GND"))
 (segment (start 136.85 130.675) (end 135.991542 131.533458) (width 0.5) (layer "F.Cu") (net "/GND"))
 (segment (start 134.4704 132.715) (end 135.45 133.6946) (width 0.5) (layer "F.Cu") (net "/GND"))
 (segment (start 127.775 129.875) (end 127.0538 130.5962) (width 0.3) (layer "F.Cu") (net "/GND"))
 (segment (start 133.4704 132.75) (end 133.4704 132.715) (width 0.25) (layer "F.Cu") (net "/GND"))
 (segment (start 133.802082 136.55) (end 135.301041 135.051041) (width 0.3) (layer "F.Cu") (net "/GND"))
 (segment (start 132.883458 131.533458) (end 131.975 130.625) (width 0.5) (layer "F.Cu") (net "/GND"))
 (segment (start 122.688201 135.325) (end 120.8532 133.489999) (width 0.3) (layer "F.Cu") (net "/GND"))
 (segment (start 135.45 134.902082) (end 135.301041 135.051041) (width 0.5) (layer "F.Cu") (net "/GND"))
 (segment (start 123.877906 135.325) (end 122.688201 135.325) (width 0.3) (layer "F.Cu") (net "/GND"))
 (segment (start 127.0538 130.5962) (end 127.0538 132.149106) (width 0.3) (layer "F.Cu") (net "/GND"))
 (segment (start 127.775 132.727082) (end 129.836459 134.788541) (width 0.3) (layer "F.Cu") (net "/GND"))
 (segment (start 127.775 128.7762) (end 127.5538 128.7762) (width 0.3) (layer "F.Cu") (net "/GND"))
 (segment (start 129.15 130.828154) (end 129.15 130.875) (width 0.3) (layer "F.Cu") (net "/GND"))
 (segment (start 132.155399 130.625) (end 131.975 130.625) (width 0.5) (layer "F.Cu") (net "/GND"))
 (segment (start 134.4704 132.715) (end 133.4704 132.715) (width 0.5) (layer "F.Cu") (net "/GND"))
 (segment (start 135.991542 131.533458) (end 132.883458 131.533458) (width 0.5) (layer "F.Cu") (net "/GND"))
 (segment (start 128.0538 128.7762) (end 127.775 128.7762) (width 0.3) (layer "F.Cu") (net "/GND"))
 (segment (start 127.0538 132.149106) (end 123.877906 135.325) (width 0.3) (layer "F.Cu") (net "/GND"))
 (segment (start 127.775 129.875) (end 127.775 129.975) (width 0.3) (layer "F.Cu") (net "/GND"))
 (segment (start 135.301041 135.051041) (end 134.876041 135.051041) (width 0.5) (layer "F.Cu") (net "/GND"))
 (segment (start 134.7854 132.4) (end 134.4704 132.715) (width 0.5) (layer "F.Cu") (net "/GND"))
 (segment (start 131.597918 136.55) (end 133.802082 136.55) (width 0.3) (layer "F.Cu") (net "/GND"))
 (segment (start 131.975 130.625) (end 132.008084 130.625) (width 0.5) (layer "F.Cu") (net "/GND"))
 (segment (start 129.836459 134.788541) (end 131.597918 136.55) (width 0.3) (layer "F.Cu") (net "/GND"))
 (segment (start 135.45 133.6946) (end 135.45 134.902082) (width 0.5) (layer "F.Cu") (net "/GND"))
 (segment (start 134.876041 135.051041) (end 133.4704 133.6454) (width 0.5) (layer "F.Cu") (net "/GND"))
 (segment (start 128.196846 129.875) (end 129.15 130.828154) (width 0.3) (layer "F.Cu") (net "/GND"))
 (segment (start 120.8532 133.489999) (end 120.8532 132.715) (width 0.3) (layer "F.Cu") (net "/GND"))
 (segment (start 135.475 132.4) (end 134.7854 132.4) (width 0.5) (layer "F.Cu") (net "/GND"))
 (segment (start 127.585 130.065) (end 127.775 129.875) (width 0.25) (layer "F.Cu") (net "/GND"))
 (segment (start 127.775 128.7762) (end 127.775 129.875) (width 0.3) (layer "F.Cu") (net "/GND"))
 (segment (start 127.775 129.875) (end 128.196846 129.875) (width 0.3) (layer "F.Cu") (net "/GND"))
 (segment (start 133.4704 133.6454) (end 133.4704 132.715) (width 0.5) (layer "F.Cu") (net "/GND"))
 (segment (start 134.325 127.55) (end 136.375 129.6) (width 0.5) (layer "F.Cu") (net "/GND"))
 (segment (start 132.008084 130.625) (end 133.4704 132.087316) (width 0.5) (layer "F.Cu") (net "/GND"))
 (via (at 127.775 129.875) (size 0.8) (drill 0.4) (layers "F.Cu" "B.Cu") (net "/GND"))
 (via (at 136.375 129.6) (size 0.8) (drill 0.4) (layers "F.Cu" "B.Cu") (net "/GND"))
 (via (at 127.775 132.727082) (size 0.8) (drill 0.4) (layers "F.Cu" "B.Cu") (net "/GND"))
 (via (at 135.475 132.4) (size 0.8) (drill 0.4) (layers "F.Cu" "B.Cu") (capping no) (covering (front no) (back no))
  (plugging (front no) (back no)) (filling no) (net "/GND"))
 (via (at 135.301041 135.051041) (size 0.8) (drill 0.4) (layers "F.Cu" "B.Cu") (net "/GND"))
 (via (at 136.85 130.675) (size 0.8) (drill 0.4) (layers "F.Cu" "B.Cu") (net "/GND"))
 (segment (start 127.775 132.727082) (end 127.775 129.875) (width 0.5) (layer "B.Cu") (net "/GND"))
 (segment (start 136.85 130.075) (end 136.375 129.6) (width 0.5) (layer "B.Cu") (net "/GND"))
 (segment (start 135.475 134.877082) (end 135.301041 135.051041) (width 0.5) (layer "B.Cu") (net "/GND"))
 (segment (start 136.85 130.675) (end 136.85 130.075) (width 0.5) (layer "B.Cu") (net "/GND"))
 (segment (start 135.475 132.05) (end 136.85 130.675) (width 0.5) (layer "B.Cu") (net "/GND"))
 (segment (start 135.425 130.55) (end 135.425 132.35) (width 0.5) (layer "B.Cu") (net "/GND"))
 (segment (start 135.475 132.4) (end 135.475 134.877082) (width 0.5) (layer "B.Cu") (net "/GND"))
 (segment (start 136.375 129.6) (end 135.425 130.55) (width 0.5) (layer "B.Cu") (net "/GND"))
 (segment (start 135.475 132.4) (end 135.475 132.05) (width 0.5) (layer "B.Cu") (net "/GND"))
 (segment (start 135.425 132.35) (end 135.475 132.4) (width 0.5) (layer "B.Cu") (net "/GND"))
 (segment (start 123.9774 134.5184) (end 122.9868 134.5184) (width 0.3) (layer "F.Cu") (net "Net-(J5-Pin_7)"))
 (segment (start 126.5538 128.7762) (end 126.5538 131.942) (width 0.3) (layer "F.Cu") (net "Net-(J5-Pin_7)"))
 (segment (start 122.8852 132.747) (end 122.8532 132.715) (width 0.25) (layer "F.Cu") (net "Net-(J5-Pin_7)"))
 (segment (start 122.8852 134.4168) (end 122.8852 132.747) (width 0.3) (layer "F.Cu") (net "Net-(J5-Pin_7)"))
 (segment (start 122.9868 134.5184) (end 122.8852 134.4168) (width 0.3) (layer "F.Cu") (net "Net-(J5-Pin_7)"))
 (segment (start 126.5538 131.942) (end 123.9774 134.5184) (width 0.3) (layer "F.Cu") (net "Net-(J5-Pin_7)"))
 (segment (start 126.0538 130.5144) (end 123.8532 132.715) (width 0.3) (layer "F.Cu") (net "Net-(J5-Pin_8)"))
 (segment (start 126.0538 128.7762) (end 126.0538 130.5144) (width 0.3) (layer "F.Cu") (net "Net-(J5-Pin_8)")))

